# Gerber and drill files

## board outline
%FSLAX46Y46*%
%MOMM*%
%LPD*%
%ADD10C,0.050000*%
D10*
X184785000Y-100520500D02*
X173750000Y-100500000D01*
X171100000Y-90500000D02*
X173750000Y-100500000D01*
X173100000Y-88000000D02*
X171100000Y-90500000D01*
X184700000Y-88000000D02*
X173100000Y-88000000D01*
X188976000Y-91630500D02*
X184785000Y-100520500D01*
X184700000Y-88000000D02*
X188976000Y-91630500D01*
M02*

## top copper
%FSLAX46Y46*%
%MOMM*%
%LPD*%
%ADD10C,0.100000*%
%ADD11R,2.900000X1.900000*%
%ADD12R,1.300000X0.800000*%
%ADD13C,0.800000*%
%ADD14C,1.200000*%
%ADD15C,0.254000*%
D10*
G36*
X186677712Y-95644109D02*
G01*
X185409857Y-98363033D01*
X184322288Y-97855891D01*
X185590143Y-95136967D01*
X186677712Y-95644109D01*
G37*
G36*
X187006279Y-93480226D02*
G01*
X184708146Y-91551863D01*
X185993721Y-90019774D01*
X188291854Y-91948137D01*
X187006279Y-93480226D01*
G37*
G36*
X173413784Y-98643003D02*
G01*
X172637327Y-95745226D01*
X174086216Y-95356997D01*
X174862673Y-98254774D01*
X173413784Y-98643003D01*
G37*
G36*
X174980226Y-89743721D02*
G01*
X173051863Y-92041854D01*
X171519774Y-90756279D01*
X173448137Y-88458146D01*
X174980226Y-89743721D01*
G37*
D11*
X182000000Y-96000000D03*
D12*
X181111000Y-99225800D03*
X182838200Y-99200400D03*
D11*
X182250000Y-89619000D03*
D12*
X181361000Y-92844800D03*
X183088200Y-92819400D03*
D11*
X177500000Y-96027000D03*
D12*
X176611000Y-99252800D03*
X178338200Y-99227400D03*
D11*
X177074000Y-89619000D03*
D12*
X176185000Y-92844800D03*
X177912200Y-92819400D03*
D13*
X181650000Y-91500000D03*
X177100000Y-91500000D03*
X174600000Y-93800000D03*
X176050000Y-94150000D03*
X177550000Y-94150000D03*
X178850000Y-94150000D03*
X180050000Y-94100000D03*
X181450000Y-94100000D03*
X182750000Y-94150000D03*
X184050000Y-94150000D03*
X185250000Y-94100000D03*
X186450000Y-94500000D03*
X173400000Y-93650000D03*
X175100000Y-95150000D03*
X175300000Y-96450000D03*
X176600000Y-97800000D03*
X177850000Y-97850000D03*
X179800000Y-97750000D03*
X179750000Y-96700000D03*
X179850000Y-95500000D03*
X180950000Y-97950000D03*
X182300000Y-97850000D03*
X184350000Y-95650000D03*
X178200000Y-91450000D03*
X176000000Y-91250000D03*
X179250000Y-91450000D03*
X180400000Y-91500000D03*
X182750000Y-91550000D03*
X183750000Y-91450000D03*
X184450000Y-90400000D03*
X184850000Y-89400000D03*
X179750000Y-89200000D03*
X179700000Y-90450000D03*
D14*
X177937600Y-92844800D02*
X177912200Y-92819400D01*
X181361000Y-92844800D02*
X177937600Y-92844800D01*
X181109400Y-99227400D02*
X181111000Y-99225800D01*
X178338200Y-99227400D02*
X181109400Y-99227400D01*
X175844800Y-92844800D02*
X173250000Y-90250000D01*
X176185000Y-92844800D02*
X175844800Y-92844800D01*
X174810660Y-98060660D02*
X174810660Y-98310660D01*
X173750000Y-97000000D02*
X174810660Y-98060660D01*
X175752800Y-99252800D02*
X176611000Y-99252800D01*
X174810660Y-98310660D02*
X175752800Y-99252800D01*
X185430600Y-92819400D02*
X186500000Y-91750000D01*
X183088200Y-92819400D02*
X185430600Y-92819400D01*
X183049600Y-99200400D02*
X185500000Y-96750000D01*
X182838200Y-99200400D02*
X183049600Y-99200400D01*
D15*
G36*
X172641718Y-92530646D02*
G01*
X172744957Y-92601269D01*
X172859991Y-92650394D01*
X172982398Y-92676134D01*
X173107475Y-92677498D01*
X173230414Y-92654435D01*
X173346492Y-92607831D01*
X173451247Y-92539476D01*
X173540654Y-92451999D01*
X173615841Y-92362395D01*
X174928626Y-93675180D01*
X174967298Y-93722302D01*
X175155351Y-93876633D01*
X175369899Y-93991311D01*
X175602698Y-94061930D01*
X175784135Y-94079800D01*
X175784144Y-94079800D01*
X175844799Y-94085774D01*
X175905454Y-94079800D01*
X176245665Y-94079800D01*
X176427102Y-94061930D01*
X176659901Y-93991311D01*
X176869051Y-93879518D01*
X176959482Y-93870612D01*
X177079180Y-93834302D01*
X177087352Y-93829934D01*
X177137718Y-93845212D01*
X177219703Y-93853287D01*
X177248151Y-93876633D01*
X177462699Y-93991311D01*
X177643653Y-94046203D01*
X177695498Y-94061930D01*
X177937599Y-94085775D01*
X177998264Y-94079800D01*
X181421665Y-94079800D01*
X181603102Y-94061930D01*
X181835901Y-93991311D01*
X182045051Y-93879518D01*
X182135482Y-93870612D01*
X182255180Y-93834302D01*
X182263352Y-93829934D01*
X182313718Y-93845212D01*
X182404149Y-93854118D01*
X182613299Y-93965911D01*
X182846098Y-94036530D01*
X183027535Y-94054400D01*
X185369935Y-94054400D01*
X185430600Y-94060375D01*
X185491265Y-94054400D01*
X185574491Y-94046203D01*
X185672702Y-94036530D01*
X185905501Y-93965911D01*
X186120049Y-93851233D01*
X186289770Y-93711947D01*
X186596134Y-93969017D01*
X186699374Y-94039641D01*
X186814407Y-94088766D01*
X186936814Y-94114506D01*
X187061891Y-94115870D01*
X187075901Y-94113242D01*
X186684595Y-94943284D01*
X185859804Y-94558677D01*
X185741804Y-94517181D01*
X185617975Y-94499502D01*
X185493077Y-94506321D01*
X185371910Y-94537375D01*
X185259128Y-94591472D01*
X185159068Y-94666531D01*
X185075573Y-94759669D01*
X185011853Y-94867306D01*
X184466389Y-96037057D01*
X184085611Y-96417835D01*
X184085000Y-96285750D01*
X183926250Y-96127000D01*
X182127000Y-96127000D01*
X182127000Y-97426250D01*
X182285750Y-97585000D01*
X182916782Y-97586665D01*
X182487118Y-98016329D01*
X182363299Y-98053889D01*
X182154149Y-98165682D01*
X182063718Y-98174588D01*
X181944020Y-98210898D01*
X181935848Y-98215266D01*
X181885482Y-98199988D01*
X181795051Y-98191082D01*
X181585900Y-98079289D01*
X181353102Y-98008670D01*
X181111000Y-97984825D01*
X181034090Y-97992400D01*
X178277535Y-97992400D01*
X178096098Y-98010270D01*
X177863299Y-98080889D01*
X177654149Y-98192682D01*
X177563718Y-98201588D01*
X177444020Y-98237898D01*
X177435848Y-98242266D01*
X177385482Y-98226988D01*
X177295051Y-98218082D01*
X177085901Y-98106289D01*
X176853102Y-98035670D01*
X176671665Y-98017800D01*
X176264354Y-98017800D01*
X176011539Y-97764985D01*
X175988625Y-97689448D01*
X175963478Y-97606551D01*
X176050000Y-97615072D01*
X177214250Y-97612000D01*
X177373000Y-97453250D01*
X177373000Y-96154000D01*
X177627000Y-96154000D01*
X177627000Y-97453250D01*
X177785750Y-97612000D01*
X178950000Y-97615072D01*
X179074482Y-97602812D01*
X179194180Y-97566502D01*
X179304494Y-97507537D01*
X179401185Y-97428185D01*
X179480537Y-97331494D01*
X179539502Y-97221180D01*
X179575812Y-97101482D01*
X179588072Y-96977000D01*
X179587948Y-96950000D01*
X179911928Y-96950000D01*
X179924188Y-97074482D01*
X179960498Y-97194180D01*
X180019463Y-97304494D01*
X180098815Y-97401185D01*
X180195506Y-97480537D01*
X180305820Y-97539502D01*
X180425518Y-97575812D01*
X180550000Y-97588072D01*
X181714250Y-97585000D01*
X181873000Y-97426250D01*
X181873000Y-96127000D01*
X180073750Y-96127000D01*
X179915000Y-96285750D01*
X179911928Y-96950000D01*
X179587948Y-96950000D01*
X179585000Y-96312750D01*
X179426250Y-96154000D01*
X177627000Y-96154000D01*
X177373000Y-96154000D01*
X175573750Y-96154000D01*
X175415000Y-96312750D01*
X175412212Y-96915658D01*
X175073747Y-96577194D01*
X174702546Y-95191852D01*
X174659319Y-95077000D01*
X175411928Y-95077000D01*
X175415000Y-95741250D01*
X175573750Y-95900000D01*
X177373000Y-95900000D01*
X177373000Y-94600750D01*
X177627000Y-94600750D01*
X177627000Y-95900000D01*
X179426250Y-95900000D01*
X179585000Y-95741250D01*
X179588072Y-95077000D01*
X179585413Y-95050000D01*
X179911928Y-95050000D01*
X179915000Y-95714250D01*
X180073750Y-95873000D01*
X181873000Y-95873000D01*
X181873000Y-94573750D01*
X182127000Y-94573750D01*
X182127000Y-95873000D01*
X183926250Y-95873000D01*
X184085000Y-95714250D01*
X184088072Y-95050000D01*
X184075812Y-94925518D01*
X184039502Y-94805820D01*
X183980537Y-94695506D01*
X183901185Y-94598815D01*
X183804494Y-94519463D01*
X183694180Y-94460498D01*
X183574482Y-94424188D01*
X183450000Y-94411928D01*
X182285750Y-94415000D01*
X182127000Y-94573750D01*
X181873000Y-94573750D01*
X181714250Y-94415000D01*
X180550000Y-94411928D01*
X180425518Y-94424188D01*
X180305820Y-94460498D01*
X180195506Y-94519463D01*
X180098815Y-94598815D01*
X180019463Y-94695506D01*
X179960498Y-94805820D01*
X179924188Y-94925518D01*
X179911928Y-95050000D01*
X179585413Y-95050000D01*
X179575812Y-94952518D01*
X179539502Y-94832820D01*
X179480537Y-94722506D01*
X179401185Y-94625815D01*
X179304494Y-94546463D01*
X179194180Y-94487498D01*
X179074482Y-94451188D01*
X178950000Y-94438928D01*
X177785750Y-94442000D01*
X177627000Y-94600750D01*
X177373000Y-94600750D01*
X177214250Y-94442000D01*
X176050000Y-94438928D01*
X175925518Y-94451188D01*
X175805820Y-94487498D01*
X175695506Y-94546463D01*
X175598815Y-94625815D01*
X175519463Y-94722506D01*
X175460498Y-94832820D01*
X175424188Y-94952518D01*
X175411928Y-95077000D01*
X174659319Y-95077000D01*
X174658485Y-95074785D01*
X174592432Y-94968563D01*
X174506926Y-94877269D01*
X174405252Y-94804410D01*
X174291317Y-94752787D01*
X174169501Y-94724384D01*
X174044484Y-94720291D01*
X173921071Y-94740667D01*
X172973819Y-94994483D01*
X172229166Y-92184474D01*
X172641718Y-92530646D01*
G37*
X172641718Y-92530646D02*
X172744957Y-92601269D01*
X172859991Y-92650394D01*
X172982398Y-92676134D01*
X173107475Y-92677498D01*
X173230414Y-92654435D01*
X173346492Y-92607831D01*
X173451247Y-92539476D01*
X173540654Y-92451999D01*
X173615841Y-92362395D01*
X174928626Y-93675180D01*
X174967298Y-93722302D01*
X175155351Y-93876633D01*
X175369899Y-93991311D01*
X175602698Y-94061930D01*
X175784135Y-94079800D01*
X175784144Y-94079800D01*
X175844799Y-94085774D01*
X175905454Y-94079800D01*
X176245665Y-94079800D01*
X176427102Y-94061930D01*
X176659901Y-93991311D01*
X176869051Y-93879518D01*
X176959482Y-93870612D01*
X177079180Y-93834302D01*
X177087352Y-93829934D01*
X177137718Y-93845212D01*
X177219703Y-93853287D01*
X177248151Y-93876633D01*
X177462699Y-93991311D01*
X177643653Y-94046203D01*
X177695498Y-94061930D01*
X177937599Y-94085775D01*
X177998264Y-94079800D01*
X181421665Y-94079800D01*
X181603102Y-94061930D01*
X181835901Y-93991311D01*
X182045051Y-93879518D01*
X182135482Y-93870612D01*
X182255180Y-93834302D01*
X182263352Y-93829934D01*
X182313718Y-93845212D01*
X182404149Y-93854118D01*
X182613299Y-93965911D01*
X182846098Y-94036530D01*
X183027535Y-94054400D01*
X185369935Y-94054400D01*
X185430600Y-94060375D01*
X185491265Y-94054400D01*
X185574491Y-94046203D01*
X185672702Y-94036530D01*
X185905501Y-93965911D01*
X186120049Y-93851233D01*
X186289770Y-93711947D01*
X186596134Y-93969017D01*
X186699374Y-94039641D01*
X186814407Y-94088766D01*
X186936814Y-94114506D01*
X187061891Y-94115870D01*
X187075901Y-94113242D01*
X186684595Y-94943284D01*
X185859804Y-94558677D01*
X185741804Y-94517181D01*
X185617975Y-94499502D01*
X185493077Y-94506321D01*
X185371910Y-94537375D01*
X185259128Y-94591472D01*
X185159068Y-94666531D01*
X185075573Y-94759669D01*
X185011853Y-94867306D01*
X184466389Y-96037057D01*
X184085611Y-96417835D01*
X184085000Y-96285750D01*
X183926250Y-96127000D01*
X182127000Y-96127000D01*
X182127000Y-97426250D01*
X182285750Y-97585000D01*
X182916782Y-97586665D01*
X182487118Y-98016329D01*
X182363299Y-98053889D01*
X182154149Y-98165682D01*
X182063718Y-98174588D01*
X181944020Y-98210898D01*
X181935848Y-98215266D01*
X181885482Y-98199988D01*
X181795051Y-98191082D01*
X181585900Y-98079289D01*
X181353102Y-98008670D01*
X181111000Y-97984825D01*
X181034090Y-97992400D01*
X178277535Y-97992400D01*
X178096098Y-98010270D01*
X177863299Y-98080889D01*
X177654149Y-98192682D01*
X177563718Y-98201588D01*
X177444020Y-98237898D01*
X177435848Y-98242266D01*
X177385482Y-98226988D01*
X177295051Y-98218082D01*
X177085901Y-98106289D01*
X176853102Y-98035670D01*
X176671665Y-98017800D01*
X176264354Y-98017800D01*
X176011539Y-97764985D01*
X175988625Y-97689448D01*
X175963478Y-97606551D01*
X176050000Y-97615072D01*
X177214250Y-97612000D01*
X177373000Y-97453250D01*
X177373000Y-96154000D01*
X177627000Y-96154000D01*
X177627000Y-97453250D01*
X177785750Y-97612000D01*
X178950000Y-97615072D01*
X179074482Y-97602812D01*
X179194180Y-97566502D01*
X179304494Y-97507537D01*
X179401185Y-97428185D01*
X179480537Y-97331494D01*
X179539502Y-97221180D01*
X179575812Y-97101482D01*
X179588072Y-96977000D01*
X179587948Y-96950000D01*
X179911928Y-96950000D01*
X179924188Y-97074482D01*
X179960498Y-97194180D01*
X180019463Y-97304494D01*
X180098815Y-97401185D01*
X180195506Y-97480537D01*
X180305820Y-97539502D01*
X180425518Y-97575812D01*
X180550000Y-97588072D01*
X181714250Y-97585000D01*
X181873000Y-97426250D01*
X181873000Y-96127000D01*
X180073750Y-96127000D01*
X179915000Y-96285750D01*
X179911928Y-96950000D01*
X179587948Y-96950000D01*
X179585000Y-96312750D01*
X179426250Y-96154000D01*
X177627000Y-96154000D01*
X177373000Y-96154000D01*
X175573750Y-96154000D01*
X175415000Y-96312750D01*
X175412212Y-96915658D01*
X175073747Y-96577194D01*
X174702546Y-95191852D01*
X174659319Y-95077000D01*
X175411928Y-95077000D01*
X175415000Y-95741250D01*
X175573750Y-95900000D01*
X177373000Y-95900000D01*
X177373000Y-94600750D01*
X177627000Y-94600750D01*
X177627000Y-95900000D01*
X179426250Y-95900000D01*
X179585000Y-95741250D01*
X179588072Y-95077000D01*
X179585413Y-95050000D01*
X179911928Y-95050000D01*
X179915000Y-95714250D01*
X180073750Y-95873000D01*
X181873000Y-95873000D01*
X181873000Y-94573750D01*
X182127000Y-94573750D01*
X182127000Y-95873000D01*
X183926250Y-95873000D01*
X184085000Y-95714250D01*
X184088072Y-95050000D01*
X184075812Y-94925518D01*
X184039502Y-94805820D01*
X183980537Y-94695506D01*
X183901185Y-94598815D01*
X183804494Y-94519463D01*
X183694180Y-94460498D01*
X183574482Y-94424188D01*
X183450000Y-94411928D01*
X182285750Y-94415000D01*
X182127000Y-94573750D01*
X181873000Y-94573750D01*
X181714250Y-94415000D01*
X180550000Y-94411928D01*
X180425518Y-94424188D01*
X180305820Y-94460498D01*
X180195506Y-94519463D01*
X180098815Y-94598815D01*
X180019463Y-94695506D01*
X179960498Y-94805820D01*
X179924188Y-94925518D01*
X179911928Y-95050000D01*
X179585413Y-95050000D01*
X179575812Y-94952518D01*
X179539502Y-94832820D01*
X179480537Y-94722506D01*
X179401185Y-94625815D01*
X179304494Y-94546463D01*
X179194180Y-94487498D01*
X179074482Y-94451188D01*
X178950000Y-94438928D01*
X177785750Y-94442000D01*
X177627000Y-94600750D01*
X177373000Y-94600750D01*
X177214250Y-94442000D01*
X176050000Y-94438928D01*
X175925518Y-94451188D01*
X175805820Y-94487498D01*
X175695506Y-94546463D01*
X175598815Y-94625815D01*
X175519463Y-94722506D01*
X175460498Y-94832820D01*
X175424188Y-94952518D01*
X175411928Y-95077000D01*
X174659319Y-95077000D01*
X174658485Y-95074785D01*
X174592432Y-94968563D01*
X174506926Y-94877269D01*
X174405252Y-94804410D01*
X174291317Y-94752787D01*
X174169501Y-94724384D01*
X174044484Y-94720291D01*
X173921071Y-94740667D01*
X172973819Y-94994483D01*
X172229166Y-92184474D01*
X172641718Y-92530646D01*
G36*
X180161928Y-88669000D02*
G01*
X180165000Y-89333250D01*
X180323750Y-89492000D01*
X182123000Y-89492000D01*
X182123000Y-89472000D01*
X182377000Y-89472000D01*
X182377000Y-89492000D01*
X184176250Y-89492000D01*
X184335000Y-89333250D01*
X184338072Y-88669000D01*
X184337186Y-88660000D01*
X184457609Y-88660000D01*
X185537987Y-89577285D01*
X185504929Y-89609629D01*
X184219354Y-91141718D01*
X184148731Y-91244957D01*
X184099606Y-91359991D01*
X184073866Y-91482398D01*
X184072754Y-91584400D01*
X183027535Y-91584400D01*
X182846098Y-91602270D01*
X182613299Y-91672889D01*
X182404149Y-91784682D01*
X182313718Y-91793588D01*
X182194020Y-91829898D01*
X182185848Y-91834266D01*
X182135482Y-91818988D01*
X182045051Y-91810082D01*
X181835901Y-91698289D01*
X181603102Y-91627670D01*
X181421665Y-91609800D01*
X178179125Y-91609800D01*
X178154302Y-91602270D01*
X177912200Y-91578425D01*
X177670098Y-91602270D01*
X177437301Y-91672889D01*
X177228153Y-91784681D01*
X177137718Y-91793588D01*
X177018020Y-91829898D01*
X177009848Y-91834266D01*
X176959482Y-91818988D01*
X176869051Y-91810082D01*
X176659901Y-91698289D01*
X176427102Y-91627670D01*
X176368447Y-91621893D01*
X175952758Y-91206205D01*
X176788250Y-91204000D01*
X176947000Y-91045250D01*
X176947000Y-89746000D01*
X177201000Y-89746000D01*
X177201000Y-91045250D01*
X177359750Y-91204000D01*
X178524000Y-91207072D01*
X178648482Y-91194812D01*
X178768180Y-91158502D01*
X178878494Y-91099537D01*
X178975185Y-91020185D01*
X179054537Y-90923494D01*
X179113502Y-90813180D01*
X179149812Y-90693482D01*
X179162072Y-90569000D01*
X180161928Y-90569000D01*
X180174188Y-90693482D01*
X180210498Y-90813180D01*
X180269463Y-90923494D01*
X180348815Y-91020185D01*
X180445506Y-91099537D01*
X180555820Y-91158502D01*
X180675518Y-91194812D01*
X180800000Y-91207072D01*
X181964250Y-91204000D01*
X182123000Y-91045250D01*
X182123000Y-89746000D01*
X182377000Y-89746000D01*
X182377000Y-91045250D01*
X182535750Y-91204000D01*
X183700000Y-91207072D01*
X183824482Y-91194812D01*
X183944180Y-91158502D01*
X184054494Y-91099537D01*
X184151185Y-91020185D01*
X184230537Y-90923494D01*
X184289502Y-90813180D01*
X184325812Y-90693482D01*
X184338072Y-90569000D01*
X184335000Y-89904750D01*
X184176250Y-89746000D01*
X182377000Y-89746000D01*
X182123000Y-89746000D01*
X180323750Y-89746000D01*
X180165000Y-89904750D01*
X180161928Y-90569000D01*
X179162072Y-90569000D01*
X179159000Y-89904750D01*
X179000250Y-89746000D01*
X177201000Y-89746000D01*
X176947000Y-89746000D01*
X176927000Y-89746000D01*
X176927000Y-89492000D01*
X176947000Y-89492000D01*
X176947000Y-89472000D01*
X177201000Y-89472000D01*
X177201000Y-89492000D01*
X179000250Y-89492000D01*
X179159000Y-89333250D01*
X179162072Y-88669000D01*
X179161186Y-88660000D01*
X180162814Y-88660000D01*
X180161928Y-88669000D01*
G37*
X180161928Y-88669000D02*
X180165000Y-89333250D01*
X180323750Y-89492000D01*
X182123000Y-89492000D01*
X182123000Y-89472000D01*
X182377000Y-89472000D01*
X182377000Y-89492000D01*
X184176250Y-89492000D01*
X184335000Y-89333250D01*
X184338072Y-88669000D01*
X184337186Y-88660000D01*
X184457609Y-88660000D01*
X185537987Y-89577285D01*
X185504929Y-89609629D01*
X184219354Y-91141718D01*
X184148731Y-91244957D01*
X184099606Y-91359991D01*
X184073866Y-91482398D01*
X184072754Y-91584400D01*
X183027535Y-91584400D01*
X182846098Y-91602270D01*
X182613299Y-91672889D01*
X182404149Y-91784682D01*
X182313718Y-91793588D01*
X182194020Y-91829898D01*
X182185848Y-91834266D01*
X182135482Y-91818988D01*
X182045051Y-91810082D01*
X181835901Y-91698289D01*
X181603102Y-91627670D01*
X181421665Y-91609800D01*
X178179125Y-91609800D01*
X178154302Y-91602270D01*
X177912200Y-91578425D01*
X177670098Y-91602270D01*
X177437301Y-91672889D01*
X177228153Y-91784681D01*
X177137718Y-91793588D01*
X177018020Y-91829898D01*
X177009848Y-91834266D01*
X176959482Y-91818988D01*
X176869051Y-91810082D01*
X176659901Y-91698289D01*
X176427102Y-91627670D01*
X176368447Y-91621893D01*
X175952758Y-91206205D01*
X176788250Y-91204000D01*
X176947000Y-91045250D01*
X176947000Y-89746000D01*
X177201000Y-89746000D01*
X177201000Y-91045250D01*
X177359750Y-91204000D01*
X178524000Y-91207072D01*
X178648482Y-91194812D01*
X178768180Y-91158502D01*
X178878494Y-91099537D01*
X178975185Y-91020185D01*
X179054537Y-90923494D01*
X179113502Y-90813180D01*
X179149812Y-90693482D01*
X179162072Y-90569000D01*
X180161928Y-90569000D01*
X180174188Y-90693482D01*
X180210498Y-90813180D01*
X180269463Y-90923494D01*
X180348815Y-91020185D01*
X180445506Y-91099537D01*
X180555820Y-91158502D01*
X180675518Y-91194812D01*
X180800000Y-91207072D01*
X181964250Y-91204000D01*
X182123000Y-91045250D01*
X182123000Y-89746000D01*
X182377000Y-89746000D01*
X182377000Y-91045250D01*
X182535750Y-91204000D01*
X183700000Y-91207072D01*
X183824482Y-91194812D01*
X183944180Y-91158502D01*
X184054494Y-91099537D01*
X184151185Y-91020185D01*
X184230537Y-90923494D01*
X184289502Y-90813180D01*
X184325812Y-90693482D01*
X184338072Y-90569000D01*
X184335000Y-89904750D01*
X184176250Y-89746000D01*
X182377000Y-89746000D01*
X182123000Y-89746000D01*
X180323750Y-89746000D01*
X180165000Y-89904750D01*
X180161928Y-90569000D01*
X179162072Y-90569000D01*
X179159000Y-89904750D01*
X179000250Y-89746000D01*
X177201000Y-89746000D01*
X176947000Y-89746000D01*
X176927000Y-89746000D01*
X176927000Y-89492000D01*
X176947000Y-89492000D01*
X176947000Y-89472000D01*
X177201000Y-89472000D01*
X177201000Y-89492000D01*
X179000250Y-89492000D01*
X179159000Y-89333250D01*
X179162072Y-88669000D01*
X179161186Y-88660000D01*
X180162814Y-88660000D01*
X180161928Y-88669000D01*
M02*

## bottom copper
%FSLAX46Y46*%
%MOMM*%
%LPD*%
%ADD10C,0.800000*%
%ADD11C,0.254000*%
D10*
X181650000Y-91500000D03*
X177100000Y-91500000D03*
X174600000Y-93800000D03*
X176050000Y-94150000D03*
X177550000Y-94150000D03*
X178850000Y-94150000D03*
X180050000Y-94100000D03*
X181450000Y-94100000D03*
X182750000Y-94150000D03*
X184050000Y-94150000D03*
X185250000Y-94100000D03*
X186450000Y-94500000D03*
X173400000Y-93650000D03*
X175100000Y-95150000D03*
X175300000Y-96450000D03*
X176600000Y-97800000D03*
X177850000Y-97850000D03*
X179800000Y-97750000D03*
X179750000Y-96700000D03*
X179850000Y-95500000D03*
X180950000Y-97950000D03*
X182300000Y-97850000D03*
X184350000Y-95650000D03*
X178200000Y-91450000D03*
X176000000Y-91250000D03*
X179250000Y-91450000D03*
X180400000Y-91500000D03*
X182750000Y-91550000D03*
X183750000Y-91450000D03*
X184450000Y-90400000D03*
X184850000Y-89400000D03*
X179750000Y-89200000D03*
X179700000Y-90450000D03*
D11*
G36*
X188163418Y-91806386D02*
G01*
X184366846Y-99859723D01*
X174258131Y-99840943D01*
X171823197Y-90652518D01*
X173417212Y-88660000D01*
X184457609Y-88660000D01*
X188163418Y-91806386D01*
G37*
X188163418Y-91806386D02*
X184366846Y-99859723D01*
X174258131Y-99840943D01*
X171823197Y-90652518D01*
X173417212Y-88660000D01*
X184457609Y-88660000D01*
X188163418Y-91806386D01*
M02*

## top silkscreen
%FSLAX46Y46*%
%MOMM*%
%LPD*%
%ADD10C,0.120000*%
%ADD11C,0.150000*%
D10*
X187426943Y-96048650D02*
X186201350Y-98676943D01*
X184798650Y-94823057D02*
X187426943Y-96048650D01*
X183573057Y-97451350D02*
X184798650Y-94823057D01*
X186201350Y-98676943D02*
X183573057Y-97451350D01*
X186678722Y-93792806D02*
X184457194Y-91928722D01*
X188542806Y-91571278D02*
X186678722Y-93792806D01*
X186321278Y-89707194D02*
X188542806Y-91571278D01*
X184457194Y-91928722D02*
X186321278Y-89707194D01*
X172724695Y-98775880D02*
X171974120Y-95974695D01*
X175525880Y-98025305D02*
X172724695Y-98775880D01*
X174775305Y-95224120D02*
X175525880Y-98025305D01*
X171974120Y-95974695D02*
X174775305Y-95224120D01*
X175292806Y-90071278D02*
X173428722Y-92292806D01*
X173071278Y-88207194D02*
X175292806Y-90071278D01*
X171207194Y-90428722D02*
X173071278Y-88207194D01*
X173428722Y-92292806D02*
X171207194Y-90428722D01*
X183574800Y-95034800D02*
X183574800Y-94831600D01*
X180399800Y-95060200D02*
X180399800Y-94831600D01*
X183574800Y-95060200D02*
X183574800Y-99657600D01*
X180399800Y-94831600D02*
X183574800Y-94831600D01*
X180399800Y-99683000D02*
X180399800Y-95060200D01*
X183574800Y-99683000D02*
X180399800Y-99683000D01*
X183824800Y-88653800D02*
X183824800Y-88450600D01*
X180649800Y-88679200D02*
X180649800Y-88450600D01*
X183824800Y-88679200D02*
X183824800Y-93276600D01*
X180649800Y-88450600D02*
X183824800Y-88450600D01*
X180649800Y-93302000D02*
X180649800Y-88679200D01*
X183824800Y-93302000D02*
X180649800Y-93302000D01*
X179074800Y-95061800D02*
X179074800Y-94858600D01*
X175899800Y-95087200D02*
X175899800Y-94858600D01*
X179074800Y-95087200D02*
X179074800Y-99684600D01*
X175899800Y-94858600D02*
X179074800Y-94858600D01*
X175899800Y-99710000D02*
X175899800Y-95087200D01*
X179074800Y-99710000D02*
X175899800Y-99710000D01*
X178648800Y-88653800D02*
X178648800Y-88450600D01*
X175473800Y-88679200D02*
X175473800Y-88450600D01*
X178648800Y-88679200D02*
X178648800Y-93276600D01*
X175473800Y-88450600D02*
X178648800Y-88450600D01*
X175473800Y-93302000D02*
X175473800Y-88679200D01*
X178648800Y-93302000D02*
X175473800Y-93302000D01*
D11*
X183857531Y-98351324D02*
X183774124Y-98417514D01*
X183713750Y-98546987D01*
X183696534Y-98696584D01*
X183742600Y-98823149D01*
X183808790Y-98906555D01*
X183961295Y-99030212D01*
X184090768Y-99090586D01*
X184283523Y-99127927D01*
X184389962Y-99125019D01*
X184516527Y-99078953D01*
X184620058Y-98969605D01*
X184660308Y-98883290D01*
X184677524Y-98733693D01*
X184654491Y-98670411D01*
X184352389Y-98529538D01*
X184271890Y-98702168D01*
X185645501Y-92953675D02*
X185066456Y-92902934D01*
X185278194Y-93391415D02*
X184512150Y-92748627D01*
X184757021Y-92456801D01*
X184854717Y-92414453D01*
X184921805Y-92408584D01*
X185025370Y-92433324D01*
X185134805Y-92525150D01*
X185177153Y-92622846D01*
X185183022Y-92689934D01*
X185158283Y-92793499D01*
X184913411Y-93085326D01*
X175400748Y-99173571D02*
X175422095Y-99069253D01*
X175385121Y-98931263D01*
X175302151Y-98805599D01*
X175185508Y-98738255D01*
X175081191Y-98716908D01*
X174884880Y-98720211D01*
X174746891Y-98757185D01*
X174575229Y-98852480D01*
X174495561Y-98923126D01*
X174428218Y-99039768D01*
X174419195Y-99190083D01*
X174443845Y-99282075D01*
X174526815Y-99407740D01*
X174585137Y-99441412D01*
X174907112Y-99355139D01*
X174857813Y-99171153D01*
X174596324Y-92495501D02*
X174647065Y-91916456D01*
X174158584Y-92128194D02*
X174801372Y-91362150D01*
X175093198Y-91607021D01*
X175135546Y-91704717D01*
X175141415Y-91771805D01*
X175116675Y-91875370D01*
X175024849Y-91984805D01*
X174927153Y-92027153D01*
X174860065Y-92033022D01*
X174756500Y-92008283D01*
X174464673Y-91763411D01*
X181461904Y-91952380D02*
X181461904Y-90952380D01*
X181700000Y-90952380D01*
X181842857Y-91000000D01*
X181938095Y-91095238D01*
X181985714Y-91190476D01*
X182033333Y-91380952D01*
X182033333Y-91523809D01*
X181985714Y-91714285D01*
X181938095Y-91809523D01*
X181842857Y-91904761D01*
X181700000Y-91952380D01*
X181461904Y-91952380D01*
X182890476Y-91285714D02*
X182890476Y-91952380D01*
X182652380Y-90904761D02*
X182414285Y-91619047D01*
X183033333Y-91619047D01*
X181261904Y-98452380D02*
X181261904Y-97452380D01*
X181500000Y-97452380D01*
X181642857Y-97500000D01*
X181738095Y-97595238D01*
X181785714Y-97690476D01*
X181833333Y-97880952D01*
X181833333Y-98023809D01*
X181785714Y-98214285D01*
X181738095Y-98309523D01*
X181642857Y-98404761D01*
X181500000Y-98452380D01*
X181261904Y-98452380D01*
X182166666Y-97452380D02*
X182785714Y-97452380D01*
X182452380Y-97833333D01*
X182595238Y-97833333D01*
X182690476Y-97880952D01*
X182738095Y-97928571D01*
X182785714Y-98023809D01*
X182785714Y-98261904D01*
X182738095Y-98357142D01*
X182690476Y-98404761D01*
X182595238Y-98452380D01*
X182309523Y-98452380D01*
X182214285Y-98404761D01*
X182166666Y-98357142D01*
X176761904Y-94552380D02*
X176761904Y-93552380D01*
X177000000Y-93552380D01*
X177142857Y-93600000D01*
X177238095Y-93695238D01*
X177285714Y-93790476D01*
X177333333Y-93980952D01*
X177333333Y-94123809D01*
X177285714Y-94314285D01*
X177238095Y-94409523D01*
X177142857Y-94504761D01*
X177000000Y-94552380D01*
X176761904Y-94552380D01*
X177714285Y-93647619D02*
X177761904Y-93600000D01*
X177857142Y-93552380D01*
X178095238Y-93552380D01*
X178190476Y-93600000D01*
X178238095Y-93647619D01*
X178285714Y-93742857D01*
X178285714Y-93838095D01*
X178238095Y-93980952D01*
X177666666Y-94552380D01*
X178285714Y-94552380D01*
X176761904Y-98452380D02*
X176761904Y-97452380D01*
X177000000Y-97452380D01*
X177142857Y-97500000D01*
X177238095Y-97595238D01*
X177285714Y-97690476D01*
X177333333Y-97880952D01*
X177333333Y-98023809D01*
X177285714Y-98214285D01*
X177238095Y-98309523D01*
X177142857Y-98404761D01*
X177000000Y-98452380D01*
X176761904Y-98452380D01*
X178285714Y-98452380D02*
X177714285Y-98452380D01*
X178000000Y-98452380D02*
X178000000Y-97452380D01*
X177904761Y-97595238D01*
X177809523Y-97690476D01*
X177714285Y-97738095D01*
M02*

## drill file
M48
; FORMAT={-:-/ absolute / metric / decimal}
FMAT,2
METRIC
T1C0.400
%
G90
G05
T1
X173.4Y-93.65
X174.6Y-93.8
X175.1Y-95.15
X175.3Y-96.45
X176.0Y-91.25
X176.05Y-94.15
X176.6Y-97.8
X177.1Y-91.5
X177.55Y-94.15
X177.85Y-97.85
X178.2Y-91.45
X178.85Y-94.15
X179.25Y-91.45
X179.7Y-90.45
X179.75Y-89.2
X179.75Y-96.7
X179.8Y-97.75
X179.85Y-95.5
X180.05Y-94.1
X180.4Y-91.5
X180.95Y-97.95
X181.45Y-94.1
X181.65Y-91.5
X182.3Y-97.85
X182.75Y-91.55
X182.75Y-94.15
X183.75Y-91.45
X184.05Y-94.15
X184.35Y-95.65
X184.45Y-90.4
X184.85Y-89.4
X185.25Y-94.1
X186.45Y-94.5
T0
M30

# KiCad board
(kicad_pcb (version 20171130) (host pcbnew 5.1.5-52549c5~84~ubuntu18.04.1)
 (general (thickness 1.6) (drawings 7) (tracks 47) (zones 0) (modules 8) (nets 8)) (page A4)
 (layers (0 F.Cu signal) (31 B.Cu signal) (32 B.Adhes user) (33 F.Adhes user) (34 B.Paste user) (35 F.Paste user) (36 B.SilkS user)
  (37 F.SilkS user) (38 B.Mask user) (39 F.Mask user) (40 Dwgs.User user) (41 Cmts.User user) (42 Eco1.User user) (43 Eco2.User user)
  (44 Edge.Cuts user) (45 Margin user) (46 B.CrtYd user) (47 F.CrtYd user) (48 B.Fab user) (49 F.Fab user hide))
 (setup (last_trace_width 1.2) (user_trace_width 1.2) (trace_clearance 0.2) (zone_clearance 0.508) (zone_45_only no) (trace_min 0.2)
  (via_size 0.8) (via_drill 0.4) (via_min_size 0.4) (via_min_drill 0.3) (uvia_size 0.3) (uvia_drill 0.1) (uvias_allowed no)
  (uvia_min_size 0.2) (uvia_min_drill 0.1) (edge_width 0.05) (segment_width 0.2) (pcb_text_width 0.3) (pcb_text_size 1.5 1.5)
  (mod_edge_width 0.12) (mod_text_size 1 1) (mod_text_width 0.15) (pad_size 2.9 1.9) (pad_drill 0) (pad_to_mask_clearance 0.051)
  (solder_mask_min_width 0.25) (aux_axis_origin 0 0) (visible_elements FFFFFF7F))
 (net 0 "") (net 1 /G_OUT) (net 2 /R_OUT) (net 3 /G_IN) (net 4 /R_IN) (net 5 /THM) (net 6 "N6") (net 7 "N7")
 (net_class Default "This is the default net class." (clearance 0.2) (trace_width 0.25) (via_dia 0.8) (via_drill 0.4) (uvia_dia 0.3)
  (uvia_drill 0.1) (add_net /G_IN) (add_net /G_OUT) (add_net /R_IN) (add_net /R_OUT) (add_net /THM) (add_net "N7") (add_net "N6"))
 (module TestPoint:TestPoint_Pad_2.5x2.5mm (layer F.Cu) (at 185.5 96.75 155)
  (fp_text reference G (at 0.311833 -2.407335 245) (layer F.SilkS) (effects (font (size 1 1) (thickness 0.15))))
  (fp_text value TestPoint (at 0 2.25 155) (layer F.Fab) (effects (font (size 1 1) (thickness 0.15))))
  (fp_line (start -1.45 1.45) (end -1.45 -1.45) (layer F.SilkS) (width 0.12))
  (fp_line (start 1.45 1.45) (end -1.45 1.45) (layer F.SilkS) (width 0.12))
  (fp_line (start 1.45 -1.45) (end 1.45 1.45) (layer F.SilkS) (width 0.12))
  (fp_line (start -1.45 -1.45) (end 1.45 -1.45) (layer F.SilkS) (width 0.12))
  (pad 1 smd rect (at 0 0 155) (size 1.2 3) (layers F.Cu F.Mask) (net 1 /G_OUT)))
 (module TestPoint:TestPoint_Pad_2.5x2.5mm (layer F.Cu) (at 186.5 91.75 50)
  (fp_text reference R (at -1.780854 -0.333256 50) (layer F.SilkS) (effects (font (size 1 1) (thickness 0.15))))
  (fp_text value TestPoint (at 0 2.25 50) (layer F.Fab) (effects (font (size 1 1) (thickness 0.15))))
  (fp_line (start -1.45 1.45) (end -1.45 -1.45) (layer F.SilkS) (width 0.12))
  (fp_line (start 1.45 1.45) (end -1.45 1.45) (layer F.SilkS) (width 0.12))
  (fp_line (start 1.45 -1.45) (end 1.45 1.45) (layer F.SilkS) (width 0.12))
  (fp_line (start -1.45 -1.45) (end 1.45 -1.45) (layer F.SilkS) (width 0.12))
  (pad 1 smd rect (at 0 0 50) (size 2 3) (layers F.Cu F.Mask) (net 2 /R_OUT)))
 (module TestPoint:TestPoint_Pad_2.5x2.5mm (layer F.Cu) (at 173.75 97 15)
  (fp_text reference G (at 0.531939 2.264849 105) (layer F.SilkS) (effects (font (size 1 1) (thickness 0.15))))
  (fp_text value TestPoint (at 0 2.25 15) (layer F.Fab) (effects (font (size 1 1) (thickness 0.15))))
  (fp_line (start -1.45 1.45) (end -1.45 -1.45) (layer F.SilkS) (width 0.12))
  (fp_line (start 1.45 1.45) (end -1.45 1.45) (layer F.SilkS) (width 0.12))
  (fp_line (start 1.45 -1.45) (end 1.45 1.45) (layer F.SilkS) (width 0.12))
  (fp_line (start -1.45 -1.45) (end 1.45 -1.45) (layer F.SilkS) (width 0.12))
  (pad 1 smd rect (at 0 0 15) (size 1.5 3) (layers F.Cu F.Mask) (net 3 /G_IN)))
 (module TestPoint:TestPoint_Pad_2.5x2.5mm (layer F.Cu) (at 173.25 90.25 140)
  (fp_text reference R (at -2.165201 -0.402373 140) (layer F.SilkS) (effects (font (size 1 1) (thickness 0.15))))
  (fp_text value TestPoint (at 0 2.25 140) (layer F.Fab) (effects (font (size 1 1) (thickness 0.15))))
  (fp_line (start -1.45 1.45) (end -1.45 -1.45) (layer F.SilkS) (width 0.12))
  (fp_line (start 1.45 1.45) (end -1.45 1.45) (layer F.SilkS) (width 0.12))
  (fp_line (start 1.45 -1.45) (end 1.45 1.45) (layer F.SilkS) (width 0.12))
  (fp_line (start -1.45 -1.45) (end 1.45 -1.45) (layer F.SilkS) (width 0.12))
  (pad 1 smd rect (at 0 0 140) (size 2 3) (layers F.Cu F.Mask) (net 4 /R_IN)))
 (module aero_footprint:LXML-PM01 (layer F.Cu) (at 181.6698 102.223 180)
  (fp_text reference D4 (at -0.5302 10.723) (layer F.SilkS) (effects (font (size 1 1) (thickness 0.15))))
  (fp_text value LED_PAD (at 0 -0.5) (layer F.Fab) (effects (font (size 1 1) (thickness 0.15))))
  (fp_line (start -1.905 7.1882) (end -1.905 7.3914) (layer F.SilkS) (width 0.12))
  (fp_line (start 1.27 7.1628) (end 1.27 7.3914) (layer F.SilkS) (width 0.12))
  (fp_line (start -1.905 7.1628) (end -1.905 2.5654) (layer F.SilkS) (width 0.12))
  (fp_line (start 1.27 7.3914) (end -1.905 7.3914) (layer F.SilkS) (width 0.12))
  (fp_line (start 1.27 2.54) (end 1.27 7.1628) (layer F.SilkS) (width 0.12))
  (fp_line (start -1.905 2.54) (end 1.27 2.54) (layer F.SilkS) (width 0.12))
  (pad 3 smd rect (at -0.3302 6.223 180) (size 2.9 1.9) (layers F.Cu F.Mask) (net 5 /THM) (clearance 0.1))
  (pad 2 smd rect (at 0.5588 2.9972 180) (size 1.3 0.8) (layers F.Cu F.Mask) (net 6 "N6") (clearance 0.1))
  (pad 1 smd rect (at -1.1684 3.0226 180) (size 1.3 0.8) (layers F.Cu F.Mask) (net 1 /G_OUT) (clearance 0.1)))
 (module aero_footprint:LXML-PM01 (layer F.Cu) (at 181.9198 95.842 180)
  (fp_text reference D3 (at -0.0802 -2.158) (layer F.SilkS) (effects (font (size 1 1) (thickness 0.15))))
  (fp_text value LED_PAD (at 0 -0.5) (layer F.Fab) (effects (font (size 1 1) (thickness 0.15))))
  (fp_line (start -1.905 7.1882) (end -1.905 7.3914) (layer F.SilkS) (width 0.12))
  (fp_line (start 1.27 7.1628) (end 1.27 7.3914) (layer F.SilkS) (width 0.12))
  (fp_line (start -1.905 7.1628) (end -1.905 2.5654) (layer F.SilkS) (width 0.12))
  (fp_line (start 1.27 7.3914) (end -1.905 7.3914) (layer F.SilkS) (width 0.12))
  (fp_line (start 1.27 2.54) (end 1.27 7.1628) (layer F.SilkS) (width 0.12))
  (fp_line (start -1.905 2.54) (end 1.27 2.54) (layer F.SilkS) (width 0.12))
  (pad 3 smd rect (at -0.3302 6.223 180) (size 2.9 1.9) (layers F.Cu F.Mask) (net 5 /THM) (clearance 0.1))
  (pad 2 smd rect (at 0.5588 2.9972 180) (size 1.3 0.8) (layers F.Cu F.Mask) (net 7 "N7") (clearance 0.1))
  (pad 1 smd rect (at -1.1684 3.0226 180) (size 1.3 0.8) (layers F.Cu F.Mask) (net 2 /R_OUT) (clearance 0.1)))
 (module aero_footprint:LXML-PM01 (layer F.Cu) (at 177.1698 102.25 180)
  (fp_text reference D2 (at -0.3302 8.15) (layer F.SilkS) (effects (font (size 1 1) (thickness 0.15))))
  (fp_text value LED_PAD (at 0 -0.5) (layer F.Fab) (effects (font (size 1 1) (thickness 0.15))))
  (fp_line (start -1.905 7.1882) (end -1.905 7.3914) (layer F.SilkS) (width 0.12))
  (fp_line (start 1.27 7.1628) (end 1.27 7.3914) (layer F.SilkS) (width 0.12))
  (fp_line (start -1.905 7.1628) (end -1.905 2.5654) (layer F.SilkS) (width 0.12))
  (fp_line (start 1.27 7.3914) (end -1.905 7.3914) (layer F.SilkS) (width 0.12))
  (fp_line (start 1.27 2.54) (end 1.27 7.1628) (layer F.SilkS) (width 0.12))
  (fp_line (start -1.905 2.54) (end 1.27 2.54) (layer F.SilkS) (width 0.12))
  (pad 3 smd rect (at -0.3302 6.223 180) (size 2.9 1.9) (layers F.Cu F.Mask) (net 5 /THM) (clearance 0.1))
  (pad 2 smd rect (at 0.5588 2.9972 180) (size 1.3 0.8) (layers F.Cu F.Mask) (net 3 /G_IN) (clearance 0.1))
  (pad 1 smd rect (at -1.1684 3.0226 180) (size 1.3 0.8) (layers F.Cu F.Mask) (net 6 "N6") (clearance 0.1)))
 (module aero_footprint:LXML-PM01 (layer F.Cu) (at 176.7438 95.842 180)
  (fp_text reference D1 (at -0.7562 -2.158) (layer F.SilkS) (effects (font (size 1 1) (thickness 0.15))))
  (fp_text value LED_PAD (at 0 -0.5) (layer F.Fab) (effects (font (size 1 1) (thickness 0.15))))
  (fp_line (start -1.905 7.1882) (end -1.905 7.3914) (layer F.SilkS) (width 0.12))
  (fp_line (start 1.27 7.1628) (end 1.27 7.3914) (layer F.SilkS) (width 0.12))
  (fp_line (start -1.905 7.1628) (end -1.905 2.5654) (layer F.SilkS) (width 0.12))
  (fp_line (start 1.27 7.3914) (end -1.905 7.3914) (layer F.SilkS) (width 0.12))
  (fp_line (start 1.27 2.54) (end 1.27 7.1628) (layer F.SilkS) (width 0.12))
  (fp_line (start -1.905 2.54) (end 1.27 2.54) (layer F.SilkS) (width 0.12))
  (pad 3 smd rect (at -0.3302 6.223 180) (size 2.9 1.9) (layers F.Cu F.Mask) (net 5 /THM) (clearance 0.1))
  (pad 2 smd rect (at 0.5588 2.9972 180) (size 1.3 0.8) (layers F.Cu F.Mask) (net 4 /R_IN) (clearance 0.1))
  (pad 1 smd rect (at -1.1684 3.0226 180) (size 1.3 0.8) (layers F.Cu F.Mask) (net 7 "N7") (clearance 0.1)))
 (gr_line (start 184.785 100.5205) (end 173.75 100.5) (layer Edge.Cuts) (width 0.05))
 (gr_line (start 171.1 90.5) (end 173.75 100.5) (layer Edge.Cuts) (width 0.05))
 (gr_line (start 173.1 88) (end 171.1 90.5) (layer Edge.Cuts) (width 0.05))
 (gr_line (start 184.7 88) (end 173.1 88) (layer Edge.Cuts) (width 0.05))
 (gr_line (start 188.976 91.6305) (end 184.785 100.5205) (layer Edge.Cuts) (width 0.05))
 (gr_line (start 184.7 88) (end 188.976 91.6305) (layer Edge.Cuts) (width 0.05))
 (segment (start 177.9376 92.8448) (end 177.9122 92.8194) (width 1.2) (layer F.Cu) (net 7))
 (segment (start 181.361 92.8448) (end 177.9376 92.8448) (width 1.2) (layer F.Cu) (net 7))
 (segment (start 181.1094 99.2274) (end 181.111 99.2258) (width 1.2) (layer F.Cu) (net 6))
 (segment (start 178.3382 99.2274) (end 181.1094 99.2274) (width 1.2) (layer F.Cu) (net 6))
 (segment (start 175.8448 92.8448) (end 173.25 90.25) (width 1.2) (layer F.Cu) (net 4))
 (segment (start 176.185 92.8448) (end 175.8448 92.8448) (width 1.2) (layer F.Cu) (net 4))
 (segment (start 174.81066 98.06066) (end 174.81066 98.31066) (width 1.2) (layer F.Cu) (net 3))
 (segment (start 173.75 97) (end 174.81066 98.06066) (width 1.2) (layer F.Cu) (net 3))
 (segment (start 175.7528 99.2528) (end 176.611 99.2528) (width 1.2) (layer F.Cu) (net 3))
 (segment (start 174.81066 98.31066) (end 175.7528 99.2528) (width 1.2) (layer F.Cu) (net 3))
 (segment (start 185.4306 92.8194) (end 186.5 91.75) (width 1.2) (layer F.Cu) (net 2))
 (segment (start 183.0882 92.8194) (end 185.4306 92.8194) (width 1.2) (layer F.Cu) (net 2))
 (segment (start 183.0496 99.2004) (end 185.5 96.75) (width 1.2) (layer F.Cu) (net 1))
 (segment (start 182.8382 99.2004) (end 183.0496 99.2004) (width 1.2) (layer F.Cu) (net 1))
 (via (at 181.65 91.5) (size 0.8) (drill 0.4) (layers F.Cu B.Cu) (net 5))
 (via (at 177.1 91.5) (size 0.8) (drill 0.4) (layers F.Cu B.Cu) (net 5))
 (via (at 174.6 93.8) (size 0.8) (drill 0.4) (layers F.Cu B.Cu) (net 5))
 (via (at 176.05 94.15) (size 0.8) (drill 0.4) (layers F.Cu B.Cu) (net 5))
 (via (at 177.55 94.15) (size 0.8) (drill 0.4) (layers F.Cu B.Cu) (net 5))
 (via (at 178.85 94.15) (size 0.8) (drill 0.4) (layers F.Cu B.Cu) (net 5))
 (via (at 180.05 94.1) (size 0.8) (drill 0.4) (layers F.Cu B.Cu) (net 5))
 (via (at 181.45 94.1) (size 0.8) (drill 0.4) (layers F.Cu B.Cu) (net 5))
 (via (at 182.75 94.15) (size 0.8) (drill 0.4) (layers F.Cu B.Cu) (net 5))
 (via (at 184.05 94.15) (size 0.8) (drill 0.4) (layers F.Cu B.Cu) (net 5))
 (via (at 185.25 94.1) (size 0.8) (drill 0.4) (layers F.Cu B.Cu) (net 5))
 (via (at 186.45 94.5) (size 0.8) (drill 0.4) (layers F.Cu B.Cu) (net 5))
 (via (at 173.4 93.65) (size 0.8) (drill 0.4) (layers F.Cu B.Cu) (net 5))
 (via (at 175.1 95.15) (size 0.8) (drill 0.4) (layers F.Cu B.Cu) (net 5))
 (via (at 175.3 96.45) (size 0.8) (drill 0.4) (layers F.Cu B.Cu) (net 5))
 (via (at 176.6 97.8) (size 0.8) (drill 0.4) (layers F.Cu B.Cu) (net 5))
 (via (at 177.85 97.85) (size 0.8) (drill 0.4) (layers F.Cu B.Cu) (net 5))
 (via (at 179.8 97.75) (size 0.8) (drill 0.4) (layers F.Cu B.Cu) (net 5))
 (via (at 179.75 96.7) (size 0.8) (drill 0.4) (layers F.Cu B.Cu) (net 5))
 (via (at 179.85 95.5) (size 0.8) (drill 0.4) (layers F.Cu B.Cu) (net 5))
 (via (at 180.95 97.95) (size 0.8) (drill 0.4) (layers F.Cu B.Cu) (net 5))
 (via (at 182.3 97.85) (size 0.8) (drill 0.4) (layers F.Cu B.Cu) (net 5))
 (via (at 184.35 95.65) (size 0.8) (drill 0.4) (layers F.Cu B.Cu) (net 5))
 (via (at 178.2 91.45) (size 0.8) (drill 0.4) (layers F.Cu B.Cu) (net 5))
 (via (at 176 91.25) (size 0.8) (drill 0.4) (layers F.Cu B.Cu) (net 5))
 (via (at 179.25 91.45) (size 0.8) (drill 0.4) (layers F.Cu B.Cu) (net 5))
 (via (at 180.4 91.5) (size 0.8) (drill 0.4) (layers F.Cu B.Cu) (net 5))
 (via (at 182.75 91.55) (size 0.8) (drill 0.4) (layers F.Cu B.Cu) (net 5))
 (via (at 183.75 91.45) (size 0.8) (drill 0.4) (layers F.Cu B.Cu) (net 5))
 (via (at 184.45 90.4) (size 0.8) (drill 0.4) (layers F.Cu B.Cu) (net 5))
 (via (at 184.85 89.4) (size 0.8) (drill 0.4) (layers F.Cu B.Cu) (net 5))
 (via (at 179.75 89.2) (size 0.8) (drill 0.4) (layers F.Cu B.Cu) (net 5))
 (via (at 179.7 90.45) (size 0.8) (drill 0.4) (layers F.Cu B.Cu) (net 5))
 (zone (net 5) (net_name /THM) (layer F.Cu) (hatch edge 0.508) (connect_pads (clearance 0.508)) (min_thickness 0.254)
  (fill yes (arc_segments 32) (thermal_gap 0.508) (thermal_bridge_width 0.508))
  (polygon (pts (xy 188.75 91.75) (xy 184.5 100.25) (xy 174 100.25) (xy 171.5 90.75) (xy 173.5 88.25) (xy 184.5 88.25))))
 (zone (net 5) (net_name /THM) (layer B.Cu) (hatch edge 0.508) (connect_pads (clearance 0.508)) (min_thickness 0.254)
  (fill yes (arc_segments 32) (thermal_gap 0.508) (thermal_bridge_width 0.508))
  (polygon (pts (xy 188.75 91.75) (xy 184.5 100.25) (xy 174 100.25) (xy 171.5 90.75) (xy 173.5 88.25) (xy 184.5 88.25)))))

